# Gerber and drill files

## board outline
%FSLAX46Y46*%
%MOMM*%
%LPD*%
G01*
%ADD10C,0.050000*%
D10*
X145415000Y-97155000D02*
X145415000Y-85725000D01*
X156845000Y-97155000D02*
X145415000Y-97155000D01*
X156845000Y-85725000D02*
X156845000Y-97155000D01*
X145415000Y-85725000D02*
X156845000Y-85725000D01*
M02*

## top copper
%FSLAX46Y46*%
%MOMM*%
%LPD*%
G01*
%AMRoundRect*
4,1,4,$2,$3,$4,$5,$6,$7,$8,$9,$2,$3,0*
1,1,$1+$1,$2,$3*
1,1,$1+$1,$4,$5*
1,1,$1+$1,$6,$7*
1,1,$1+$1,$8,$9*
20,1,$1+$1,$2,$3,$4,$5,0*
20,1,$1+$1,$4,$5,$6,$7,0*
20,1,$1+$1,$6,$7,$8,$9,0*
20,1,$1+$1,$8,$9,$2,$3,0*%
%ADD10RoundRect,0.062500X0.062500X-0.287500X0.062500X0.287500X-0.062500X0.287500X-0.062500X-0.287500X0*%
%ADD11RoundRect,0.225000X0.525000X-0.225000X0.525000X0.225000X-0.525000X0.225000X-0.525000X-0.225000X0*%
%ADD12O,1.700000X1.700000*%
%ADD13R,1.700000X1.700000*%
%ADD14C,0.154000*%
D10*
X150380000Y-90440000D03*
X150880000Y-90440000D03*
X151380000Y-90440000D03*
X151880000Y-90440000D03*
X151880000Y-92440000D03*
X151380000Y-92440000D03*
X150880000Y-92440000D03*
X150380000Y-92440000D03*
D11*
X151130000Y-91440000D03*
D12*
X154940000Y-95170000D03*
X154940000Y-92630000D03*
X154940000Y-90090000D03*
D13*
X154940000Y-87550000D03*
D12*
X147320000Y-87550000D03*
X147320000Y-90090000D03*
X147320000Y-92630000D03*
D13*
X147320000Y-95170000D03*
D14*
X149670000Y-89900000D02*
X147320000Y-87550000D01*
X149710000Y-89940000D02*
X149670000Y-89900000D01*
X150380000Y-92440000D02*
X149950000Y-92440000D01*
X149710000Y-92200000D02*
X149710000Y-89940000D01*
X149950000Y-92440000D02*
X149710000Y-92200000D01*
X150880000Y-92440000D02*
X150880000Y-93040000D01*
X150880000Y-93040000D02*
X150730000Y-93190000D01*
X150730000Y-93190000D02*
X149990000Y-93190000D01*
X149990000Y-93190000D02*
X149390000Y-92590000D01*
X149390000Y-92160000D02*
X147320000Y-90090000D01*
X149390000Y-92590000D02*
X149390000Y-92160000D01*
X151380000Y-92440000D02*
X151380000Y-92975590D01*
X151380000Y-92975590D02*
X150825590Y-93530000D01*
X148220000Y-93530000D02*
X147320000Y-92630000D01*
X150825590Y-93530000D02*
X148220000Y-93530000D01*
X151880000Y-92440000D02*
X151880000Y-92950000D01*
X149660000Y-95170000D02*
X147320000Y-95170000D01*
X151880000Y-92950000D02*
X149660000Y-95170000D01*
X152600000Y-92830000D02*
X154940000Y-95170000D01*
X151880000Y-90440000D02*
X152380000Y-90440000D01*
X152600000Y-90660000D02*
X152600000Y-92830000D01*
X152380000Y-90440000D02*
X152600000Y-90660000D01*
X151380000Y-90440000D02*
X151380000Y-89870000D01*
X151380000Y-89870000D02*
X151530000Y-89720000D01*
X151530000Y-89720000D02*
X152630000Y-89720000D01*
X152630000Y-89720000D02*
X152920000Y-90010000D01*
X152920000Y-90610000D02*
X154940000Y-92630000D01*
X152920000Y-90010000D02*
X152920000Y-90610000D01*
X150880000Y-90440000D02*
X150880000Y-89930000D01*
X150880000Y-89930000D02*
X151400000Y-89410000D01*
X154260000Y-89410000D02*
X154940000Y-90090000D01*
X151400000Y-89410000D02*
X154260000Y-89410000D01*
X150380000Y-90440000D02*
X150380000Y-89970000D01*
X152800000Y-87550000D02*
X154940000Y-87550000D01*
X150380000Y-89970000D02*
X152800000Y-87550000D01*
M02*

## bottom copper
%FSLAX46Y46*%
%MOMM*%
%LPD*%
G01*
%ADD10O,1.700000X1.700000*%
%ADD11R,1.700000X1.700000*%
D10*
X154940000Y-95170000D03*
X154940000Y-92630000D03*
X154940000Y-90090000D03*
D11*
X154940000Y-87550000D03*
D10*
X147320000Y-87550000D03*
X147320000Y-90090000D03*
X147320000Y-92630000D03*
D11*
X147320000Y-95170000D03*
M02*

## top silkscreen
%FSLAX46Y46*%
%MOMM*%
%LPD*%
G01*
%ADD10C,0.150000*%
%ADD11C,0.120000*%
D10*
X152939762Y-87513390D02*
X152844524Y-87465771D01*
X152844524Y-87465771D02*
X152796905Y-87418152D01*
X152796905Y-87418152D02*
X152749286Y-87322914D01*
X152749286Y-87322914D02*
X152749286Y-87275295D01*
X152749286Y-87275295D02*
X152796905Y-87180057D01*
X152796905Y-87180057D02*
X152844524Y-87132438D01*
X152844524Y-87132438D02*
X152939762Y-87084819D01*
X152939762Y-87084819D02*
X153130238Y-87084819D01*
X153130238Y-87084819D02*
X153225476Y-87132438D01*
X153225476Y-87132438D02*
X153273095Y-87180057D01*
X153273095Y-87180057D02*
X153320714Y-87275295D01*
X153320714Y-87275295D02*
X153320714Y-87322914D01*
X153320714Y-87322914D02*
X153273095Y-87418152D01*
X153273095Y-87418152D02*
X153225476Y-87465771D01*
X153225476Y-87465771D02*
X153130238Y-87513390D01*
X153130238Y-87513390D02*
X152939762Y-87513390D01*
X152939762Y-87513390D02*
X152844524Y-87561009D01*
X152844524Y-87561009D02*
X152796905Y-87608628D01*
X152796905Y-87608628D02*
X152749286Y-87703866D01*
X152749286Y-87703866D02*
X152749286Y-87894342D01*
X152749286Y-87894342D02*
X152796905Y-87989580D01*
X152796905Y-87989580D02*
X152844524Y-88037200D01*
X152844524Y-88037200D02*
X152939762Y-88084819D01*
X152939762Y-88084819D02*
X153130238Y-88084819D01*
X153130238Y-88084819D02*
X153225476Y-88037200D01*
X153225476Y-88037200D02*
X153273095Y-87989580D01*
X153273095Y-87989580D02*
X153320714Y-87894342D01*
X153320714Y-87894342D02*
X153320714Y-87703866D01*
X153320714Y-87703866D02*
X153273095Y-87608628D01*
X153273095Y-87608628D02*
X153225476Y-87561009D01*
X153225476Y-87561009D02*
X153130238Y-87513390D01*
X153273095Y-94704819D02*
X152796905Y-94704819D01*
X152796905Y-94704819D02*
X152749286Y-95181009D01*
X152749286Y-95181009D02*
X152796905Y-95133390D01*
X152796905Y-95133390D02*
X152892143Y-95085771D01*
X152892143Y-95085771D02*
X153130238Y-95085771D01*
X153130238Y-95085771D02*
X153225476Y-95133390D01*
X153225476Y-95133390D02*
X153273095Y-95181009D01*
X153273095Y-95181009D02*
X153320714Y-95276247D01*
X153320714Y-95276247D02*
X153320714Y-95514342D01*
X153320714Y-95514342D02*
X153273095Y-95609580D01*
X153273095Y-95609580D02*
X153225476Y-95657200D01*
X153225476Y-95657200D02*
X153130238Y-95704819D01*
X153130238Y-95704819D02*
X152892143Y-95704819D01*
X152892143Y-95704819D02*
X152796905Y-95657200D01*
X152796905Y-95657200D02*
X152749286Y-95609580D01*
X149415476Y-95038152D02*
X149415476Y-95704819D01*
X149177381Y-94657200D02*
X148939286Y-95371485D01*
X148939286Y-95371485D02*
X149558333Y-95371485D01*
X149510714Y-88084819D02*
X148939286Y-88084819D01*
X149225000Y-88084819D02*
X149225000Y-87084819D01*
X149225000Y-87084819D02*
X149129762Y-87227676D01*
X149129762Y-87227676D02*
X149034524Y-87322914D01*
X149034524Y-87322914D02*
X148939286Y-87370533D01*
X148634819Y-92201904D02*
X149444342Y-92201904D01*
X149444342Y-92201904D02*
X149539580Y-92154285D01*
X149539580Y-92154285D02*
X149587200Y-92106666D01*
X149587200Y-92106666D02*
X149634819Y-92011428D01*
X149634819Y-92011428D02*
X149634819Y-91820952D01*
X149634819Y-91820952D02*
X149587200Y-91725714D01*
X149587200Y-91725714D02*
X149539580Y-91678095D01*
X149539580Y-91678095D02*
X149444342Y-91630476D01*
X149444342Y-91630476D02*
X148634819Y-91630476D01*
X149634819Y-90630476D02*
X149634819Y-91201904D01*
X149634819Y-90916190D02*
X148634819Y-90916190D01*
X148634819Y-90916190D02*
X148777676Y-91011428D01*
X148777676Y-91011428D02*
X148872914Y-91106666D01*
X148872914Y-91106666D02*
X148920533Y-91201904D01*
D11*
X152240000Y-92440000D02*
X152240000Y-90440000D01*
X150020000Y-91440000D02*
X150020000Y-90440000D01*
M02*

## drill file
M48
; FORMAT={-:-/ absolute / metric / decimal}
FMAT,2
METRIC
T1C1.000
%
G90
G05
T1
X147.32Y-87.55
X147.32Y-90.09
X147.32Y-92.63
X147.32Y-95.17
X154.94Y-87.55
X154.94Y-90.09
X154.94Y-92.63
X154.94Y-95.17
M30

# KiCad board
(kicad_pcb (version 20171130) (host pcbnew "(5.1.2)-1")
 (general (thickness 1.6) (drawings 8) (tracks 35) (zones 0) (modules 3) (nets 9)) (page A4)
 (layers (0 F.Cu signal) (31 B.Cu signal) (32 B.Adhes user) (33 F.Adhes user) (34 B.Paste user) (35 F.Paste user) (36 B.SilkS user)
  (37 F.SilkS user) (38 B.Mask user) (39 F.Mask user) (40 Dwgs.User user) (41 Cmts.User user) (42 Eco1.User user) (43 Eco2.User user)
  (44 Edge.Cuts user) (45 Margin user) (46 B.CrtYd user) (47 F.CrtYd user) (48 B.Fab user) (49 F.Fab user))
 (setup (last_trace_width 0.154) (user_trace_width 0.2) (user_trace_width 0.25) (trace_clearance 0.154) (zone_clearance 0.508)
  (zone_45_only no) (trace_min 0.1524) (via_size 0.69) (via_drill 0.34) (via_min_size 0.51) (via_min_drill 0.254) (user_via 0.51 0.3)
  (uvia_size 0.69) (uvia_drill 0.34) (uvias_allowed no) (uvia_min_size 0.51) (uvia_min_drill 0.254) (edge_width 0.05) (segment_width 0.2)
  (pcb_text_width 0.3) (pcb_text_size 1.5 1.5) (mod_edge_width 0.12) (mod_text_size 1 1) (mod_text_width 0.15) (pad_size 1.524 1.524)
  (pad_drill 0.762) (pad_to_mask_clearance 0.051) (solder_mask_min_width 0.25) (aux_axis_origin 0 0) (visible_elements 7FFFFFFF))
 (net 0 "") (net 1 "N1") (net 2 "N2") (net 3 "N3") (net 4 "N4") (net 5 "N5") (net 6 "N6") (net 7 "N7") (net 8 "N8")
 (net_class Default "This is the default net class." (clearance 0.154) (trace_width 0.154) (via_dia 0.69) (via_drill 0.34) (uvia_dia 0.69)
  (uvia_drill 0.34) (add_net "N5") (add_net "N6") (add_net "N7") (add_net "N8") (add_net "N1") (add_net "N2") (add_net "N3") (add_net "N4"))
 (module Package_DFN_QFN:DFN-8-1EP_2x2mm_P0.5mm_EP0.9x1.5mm (layer F.Cu) (at 151.13 91.44 90)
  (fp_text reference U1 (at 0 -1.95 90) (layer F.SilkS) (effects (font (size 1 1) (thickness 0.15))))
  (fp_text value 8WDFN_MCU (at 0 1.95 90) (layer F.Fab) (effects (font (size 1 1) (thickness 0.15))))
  (fp_line (start -1 1.11) (end 1 1.11) (layer F.SilkS) (width 0.12))
  (fp_line (start 0 -1.11) (end 1 -1.11) (layer F.SilkS) (width 0.12))
  (pad 8 smd roundrect (at 1 -0.75 90) (size 0.7 0.25) (layers F.Cu F.Paste F.Mask) (roundrect_rratio 0.25) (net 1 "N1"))
  (pad 7 smd roundrect (at 1 -0.25 90) (size 0.7 0.25) (layers F.Cu F.Paste F.Mask) (roundrect_rratio 0.25) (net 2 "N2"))
  (pad 6 smd roundrect (at 1 0.25 90) (size 0.7 0.25) (layers F.Cu F.Paste F.Mask) (roundrect_rratio 0.25) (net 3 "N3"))
  (pad 5 smd roundrect (at 1 0.75 90) (size 0.7 0.25) (layers F.Cu F.Paste F.Mask) (roundrect_rratio 0.25) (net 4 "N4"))
  (pad 4 smd roundrect (at -1 0.75 90) (size 0.7 0.25) (layers F.Cu F.Paste F.Mask) (roundrect_rratio 0.25) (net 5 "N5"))
  (pad 3 smd roundrect (at -1 0.25 90) (size 0.7 0.25) (layers F.Cu F.Paste F.Mask) (roundrect_rratio 0.25) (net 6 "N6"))
  (pad 2 smd roundrect (at -1 -0.25 90) (size 0.7 0.25) (layers F.Cu F.Paste F.Mask) (roundrect_rratio 0.25) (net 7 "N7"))
  (pad 1 smd roundrect (at -1 -0.75 90) (size 0.7 0.25) (layers F.Cu F.Paste F.Mask) (roundrect_rratio 0.25) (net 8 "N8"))
  (pad "" smd roundrect (at 0.225 0.375 90) (size 0.36 0.6) (layers F.Paste) (roundrect_rratio 0.25))
  (pad "" smd roundrect (at 0.225 -0.375 90) (size 0.36 0.6) (layers F.Paste) (roundrect_rratio 0.25))
  (pad "" smd roundrect (at -0.225 0.375 90) (size 0.36 0.6) (layers F.Paste) (roundrect_rratio 0.25))
  (pad "" smd roundrect (at -0.225 -0.375 90) (size 0.36 0.6) (layers F.Paste) (roundrect_rratio 0.25))
  (pad 9 smd roundrect (at 0 0 90) (size 0.9 1.5) (layers F.Cu F.Mask) (roundrect_rratio 0.25)))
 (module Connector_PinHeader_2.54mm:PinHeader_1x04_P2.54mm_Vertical (layer B.Cu) (at 154.94 87.55 180)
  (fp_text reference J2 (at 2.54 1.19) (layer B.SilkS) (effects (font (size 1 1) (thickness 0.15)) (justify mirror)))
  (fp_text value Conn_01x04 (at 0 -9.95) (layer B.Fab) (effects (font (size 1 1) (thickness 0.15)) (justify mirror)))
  (pad 4 thru_hole oval (at 0 -7.62 180) (size 1.7 1.7) (drill 1) (layers *.Cu *.Mask) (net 4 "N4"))
  (pad 3 thru_hole oval (at 0 -5.08 180) (size 1.7 1.7) (drill 1) (layers *.Cu *.Mask) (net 3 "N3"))
  (pad 2 thru_hole oval (at 0 -2.54 180) (size 1.7 1.7) (drill 1) (layers *.Cu *.Mask) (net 2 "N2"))
  (pad 1 thru_hole rect (at 0 0 180) (size 1.7 1.7) (drill 1) (layers *.Cu *.Mask) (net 1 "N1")))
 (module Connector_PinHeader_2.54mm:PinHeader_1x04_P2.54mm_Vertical (layer B.Cu) (at 147.32 95.17)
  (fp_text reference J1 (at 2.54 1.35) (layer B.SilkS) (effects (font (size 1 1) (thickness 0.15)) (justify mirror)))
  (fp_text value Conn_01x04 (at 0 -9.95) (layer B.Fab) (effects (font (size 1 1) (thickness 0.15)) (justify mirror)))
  (pad 4 thru_hole oval (at 0 -7.62) (size 1.7 1.7) (drill 1) (layers *.Cu *.Mask) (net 8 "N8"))
  (pad 3 thru_hole oval (at 0 -5.08) (size 1.7 1.7) (drill 1) (layers *.Cu *.Mask) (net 7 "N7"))
  (pad 2 thru_hole oval (at 0 -2.54) (size 1.7 1.7) (drill 1) (layers *.Cu *.Mask) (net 6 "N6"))
  (pad 1 thru_hole rect (at 0 0) (size 1.7 1.7) (drill 1) (layers *.Cu *.Mask) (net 5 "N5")))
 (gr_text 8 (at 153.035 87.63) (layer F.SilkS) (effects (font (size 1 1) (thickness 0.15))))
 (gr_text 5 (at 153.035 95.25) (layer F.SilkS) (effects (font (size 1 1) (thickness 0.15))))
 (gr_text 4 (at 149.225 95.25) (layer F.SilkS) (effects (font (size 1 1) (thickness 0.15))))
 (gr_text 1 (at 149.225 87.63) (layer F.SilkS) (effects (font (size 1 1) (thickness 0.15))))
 (gr_line (start 145.415 97.155) (end 145.415 85.725) (layer Edge.Cuts) (width 0.05))
 (gr_line (start 156.845 97.155) (end 145.415 97.155) (layer Edge.Cuts) (width 0.05))
 (gr_line (start 156.845 85.725) (end 156.845 97.155) (layer Edge.Cuts) (width 0.05))
 (gr_line (start 145.415 85.725) (end 156.845 85.725) (layer Edge.Cuts) (width 0.05))
 (segment (start 149.67 89.9) (end 147.32 87.55) (width 0.154) (layer F.Cu) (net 8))
 (segment (start 149.71 89.94) (end 149.67 89.9) (width 0.154) (layer F.Cu) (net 8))
 (segment (start 150.38 92.44) (end 149.95 92.44) (width 0.154) (layer F.Cu) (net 8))
 (segment (start 149.71 92.2) (end 149.71 89.94) (width 0.154) (layer F.Cu) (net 8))
 (segment (start 149.95 92.44) (end 149.71 92.2) (width 0.154) (layer F.Cu) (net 8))
 (segment (start 150.88 92.44) (end 150.88 93.04) (width 0.154) (layer F.Cu) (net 7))
 (segment (start 150.88 93.04) (end 150.73 93.19) (width 0.154) (layer F.Cu) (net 7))
 (segment (start 150.73 93.19) (end 149.99 93.19) (width 0.154) (layer F.Cu) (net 7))
 (segment (start 149.99 93.19) (end 149.39 92.59) (width 0.154) (layer F.Cu) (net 7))
 (segment (start 149.39 92.16) (end 147.32 90.09) (width 0.154) (layer F.Cu) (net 7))
 (segment (start 149.39 92.59) (end 149.39 92.16) (width 0.154) (layer F.Cu) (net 7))
 (segment (start 151.38 92.44) (end 151.38 92.97559) (width 0.154) (layer F.Cu) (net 6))
 (segment (start 151.38 92.97559) (end 150.82559 93.53) (width 0.154) (layer F.Cu) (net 6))
 (segment (start 148.22 93.53) (end 147.32 92.63) (width 0.154) (layer F.Cu) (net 6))
 (segment (start 150.82559 93.53) (end 148.22 93.53) (width 0.154) (layer F.Cu) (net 6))
 (segment (start 151.88 92.44) (end 151.88 92.95) (width 0.154) (layer F.Cu) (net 5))
 (segment (start 149.66 95.17) (end 147.32 95.17) (width 0.154) (layer F.Cu) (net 5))
 (segment (start 151.88 92.95) (end 149.66 95.17) (width 0.154) (layer F.Cu) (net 5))
 (segment (start 152.6 92.83) (end 154.94 95.17) (width 0.154) (layer F.Cu) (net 4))
 (segment (start 151.88 90.44) (end 152.38 90.44) (width 0.154) (layer F.Cu) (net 4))
 (segment (start 152.6 90.66) (end 152.6 92.83) (width 0.154) (layer F.Cu) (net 4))
 (segment (start 152.38 90.44) (end 152.6 90.66) (width 0.154) (layer F.Cu) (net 4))
 (segment (start 151.38 90.44) (end 151.38 89.87) (width 0.154) (layer F.Cu) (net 3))
 (segment (start 151.38 89.87) (end 151.53 89.72) (width 0.154) (layer F.Cu) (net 3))
 (segment (start 151.53 89.72) (end 152.63 89.72) (width 0.154) (layer F.Cu) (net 3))
 (segment (start 152.63 89.72) (end 152.92 90.01) (width 0.154) (layer F.Cu) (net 3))
 (segment (start 152.92 90.61) (end 154.94 92.63) (width 0.154) (layer F.Cu) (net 3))
 (segment (start 152.92 90.01) (end 152.92 90.61) (width 0.154) (layer F.Cu) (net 3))
 (segment (start 150.88 90.44) (end 150.88 89.93) (width 0.154) (layer F.Cu) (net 2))
 (segment (start 150.88 89.93) (end 151.4 89.41) (width 0.154) (layer F.Cu) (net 2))
 (segment (start 154.26 89.41) (end 154.94 90.09) (width 0.154) (layer F.Cu) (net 2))
 (segment (start 151.4 89.41) (end 154.26 89.41) (width 0.154) (layer F.Cu) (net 2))
 (segment (start 150.38 90.44) (end 150.38 89.97) (width 0.154) (layer F.Cu) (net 1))
 (segment (start 152.8 87.55) (end 154.94 87.55) (width 0.154) (layer F.Cu) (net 1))
 (segment (start 150.38 89.97) (end 152.8 87.55) (width 0.154) (layer F.Cu) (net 1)))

